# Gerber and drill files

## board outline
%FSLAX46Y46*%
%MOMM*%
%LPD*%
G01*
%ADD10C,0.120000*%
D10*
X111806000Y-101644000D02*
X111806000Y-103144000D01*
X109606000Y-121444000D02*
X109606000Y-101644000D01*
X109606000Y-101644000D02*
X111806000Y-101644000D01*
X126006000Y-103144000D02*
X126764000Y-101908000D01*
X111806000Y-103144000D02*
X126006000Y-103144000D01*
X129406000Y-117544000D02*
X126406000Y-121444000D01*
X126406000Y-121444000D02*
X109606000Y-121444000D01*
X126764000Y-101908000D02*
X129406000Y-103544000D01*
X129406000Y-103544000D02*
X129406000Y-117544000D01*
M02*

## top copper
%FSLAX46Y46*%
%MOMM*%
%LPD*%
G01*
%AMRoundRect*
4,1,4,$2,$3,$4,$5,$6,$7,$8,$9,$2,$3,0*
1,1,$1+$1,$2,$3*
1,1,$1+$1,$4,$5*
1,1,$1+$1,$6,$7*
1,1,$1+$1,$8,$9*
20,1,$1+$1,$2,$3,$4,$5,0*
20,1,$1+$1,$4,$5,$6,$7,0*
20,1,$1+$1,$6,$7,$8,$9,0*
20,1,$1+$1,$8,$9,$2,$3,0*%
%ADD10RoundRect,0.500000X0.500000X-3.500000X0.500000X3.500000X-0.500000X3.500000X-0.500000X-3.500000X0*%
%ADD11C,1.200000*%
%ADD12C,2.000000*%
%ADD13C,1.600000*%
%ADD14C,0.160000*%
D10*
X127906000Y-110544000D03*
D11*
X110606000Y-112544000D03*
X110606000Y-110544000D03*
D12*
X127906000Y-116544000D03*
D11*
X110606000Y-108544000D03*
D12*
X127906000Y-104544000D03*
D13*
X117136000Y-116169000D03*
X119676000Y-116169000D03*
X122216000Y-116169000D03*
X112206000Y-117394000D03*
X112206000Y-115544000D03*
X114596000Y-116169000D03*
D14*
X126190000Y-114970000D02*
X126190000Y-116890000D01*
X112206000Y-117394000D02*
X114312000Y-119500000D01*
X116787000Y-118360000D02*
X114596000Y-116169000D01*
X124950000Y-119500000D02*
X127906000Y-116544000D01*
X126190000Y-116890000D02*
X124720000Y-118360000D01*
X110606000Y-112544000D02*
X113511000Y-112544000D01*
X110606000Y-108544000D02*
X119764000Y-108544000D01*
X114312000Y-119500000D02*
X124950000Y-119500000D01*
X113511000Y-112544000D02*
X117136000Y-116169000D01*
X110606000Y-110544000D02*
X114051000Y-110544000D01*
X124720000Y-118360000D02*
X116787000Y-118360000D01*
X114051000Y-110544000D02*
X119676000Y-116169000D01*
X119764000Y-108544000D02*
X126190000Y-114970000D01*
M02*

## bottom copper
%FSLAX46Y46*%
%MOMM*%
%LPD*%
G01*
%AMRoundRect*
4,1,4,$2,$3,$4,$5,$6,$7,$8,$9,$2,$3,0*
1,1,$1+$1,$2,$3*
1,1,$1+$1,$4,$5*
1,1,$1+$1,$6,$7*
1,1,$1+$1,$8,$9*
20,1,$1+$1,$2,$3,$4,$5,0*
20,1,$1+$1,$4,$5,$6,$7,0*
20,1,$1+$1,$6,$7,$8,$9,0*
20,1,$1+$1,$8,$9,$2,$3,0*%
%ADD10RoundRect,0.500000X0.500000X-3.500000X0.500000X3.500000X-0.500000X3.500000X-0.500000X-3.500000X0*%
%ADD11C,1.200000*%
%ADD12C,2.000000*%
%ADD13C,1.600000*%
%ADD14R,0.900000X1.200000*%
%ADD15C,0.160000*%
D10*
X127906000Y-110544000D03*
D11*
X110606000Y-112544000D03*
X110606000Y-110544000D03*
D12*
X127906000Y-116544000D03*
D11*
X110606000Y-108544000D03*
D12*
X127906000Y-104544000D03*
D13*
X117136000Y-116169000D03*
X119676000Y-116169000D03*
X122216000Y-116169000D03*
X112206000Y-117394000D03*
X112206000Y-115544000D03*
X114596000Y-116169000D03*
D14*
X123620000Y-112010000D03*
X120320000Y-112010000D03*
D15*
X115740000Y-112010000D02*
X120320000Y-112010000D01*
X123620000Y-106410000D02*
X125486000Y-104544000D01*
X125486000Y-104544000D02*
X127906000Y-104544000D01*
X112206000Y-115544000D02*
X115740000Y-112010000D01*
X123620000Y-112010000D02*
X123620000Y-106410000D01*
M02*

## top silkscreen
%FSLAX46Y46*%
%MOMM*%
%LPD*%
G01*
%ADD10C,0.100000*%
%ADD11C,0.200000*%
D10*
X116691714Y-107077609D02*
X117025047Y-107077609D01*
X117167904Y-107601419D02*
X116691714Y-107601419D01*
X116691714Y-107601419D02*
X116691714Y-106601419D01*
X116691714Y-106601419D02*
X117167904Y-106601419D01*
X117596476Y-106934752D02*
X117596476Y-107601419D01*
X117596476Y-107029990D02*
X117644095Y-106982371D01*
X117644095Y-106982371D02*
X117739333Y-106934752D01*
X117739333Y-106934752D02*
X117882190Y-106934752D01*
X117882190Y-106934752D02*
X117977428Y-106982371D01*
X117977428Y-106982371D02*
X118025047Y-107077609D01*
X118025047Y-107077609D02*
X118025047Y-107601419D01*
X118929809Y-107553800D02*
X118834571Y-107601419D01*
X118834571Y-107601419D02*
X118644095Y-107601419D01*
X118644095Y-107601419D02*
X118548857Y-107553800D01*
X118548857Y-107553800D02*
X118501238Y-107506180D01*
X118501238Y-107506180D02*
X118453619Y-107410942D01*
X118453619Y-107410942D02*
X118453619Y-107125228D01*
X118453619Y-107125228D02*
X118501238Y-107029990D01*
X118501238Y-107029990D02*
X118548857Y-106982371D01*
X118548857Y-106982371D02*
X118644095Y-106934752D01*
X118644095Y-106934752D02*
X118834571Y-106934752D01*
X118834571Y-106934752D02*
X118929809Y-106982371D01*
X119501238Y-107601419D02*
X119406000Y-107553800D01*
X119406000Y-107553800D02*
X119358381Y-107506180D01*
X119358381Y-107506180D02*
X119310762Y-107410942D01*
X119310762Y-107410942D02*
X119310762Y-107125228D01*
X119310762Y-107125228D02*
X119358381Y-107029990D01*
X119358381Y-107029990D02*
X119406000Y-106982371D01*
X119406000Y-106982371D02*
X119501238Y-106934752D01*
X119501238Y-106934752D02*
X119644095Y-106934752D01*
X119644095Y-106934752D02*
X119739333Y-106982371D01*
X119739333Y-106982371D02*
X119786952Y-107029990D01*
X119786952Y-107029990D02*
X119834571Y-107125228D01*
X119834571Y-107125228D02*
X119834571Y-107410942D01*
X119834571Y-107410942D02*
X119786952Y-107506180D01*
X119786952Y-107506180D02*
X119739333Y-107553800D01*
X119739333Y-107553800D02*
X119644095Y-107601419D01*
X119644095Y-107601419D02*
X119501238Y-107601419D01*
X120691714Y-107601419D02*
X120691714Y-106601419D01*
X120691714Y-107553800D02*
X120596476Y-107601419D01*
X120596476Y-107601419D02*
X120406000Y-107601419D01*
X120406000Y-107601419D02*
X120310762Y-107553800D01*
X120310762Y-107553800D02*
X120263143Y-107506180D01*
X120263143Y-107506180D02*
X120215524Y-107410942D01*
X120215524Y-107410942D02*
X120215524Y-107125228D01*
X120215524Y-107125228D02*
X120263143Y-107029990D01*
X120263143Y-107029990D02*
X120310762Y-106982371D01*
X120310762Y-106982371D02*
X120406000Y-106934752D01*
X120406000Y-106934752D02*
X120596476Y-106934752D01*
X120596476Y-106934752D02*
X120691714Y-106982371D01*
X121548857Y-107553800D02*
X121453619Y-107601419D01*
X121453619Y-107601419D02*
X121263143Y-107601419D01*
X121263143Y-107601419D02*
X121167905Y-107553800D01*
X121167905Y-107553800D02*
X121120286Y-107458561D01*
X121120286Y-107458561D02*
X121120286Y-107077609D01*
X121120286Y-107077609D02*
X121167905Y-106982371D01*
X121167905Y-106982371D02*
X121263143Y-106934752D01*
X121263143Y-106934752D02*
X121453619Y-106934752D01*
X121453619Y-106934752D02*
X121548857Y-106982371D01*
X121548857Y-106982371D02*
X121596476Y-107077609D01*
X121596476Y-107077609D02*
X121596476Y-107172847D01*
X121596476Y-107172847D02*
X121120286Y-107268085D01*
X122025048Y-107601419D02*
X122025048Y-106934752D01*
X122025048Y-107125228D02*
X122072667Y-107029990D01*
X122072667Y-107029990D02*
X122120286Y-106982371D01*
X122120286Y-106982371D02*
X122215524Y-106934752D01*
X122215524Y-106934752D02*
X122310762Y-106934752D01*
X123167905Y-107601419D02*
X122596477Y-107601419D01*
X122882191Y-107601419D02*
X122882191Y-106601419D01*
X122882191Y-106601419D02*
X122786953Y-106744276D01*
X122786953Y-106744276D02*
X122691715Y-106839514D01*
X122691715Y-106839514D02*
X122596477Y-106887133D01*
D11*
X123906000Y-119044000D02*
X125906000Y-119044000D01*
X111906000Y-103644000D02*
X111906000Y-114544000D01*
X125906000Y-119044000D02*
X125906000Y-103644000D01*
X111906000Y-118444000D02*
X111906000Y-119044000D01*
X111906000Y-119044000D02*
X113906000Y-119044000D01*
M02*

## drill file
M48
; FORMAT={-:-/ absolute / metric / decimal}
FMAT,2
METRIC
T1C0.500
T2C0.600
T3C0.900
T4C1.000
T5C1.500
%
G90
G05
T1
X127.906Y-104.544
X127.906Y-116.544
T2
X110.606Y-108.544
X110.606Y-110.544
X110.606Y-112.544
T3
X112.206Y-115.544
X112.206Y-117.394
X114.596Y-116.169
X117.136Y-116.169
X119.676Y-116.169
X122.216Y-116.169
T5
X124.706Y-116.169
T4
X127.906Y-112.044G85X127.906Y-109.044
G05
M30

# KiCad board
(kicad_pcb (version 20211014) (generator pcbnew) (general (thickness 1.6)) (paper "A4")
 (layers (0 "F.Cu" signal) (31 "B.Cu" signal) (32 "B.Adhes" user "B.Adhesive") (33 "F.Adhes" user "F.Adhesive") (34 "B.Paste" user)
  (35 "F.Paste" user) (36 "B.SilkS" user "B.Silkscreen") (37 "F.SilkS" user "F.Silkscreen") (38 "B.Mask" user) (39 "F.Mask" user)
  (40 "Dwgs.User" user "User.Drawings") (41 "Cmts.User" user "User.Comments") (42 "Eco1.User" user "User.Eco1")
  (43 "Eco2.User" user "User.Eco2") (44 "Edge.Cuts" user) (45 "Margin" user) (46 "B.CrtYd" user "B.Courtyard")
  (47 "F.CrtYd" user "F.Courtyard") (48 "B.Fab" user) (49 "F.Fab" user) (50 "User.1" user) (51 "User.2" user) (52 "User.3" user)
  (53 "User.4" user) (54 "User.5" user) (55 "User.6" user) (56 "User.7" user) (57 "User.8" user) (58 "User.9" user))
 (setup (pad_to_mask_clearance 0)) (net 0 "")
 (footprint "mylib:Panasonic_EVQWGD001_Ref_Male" (layer "F.Cu") (at 119.906 110.544 90)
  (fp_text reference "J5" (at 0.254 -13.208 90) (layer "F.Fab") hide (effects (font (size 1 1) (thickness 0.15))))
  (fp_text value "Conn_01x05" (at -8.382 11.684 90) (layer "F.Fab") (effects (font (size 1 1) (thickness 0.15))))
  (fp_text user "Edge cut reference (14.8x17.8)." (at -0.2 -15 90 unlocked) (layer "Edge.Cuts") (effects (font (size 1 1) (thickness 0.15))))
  (fp_line (start 8.9 -8.1) (end 7.4 -8.1) (layer "Edge.Cuts") (width 0.12))
  (fp_line (start -10.9 -10.3) (end 8.9 -10.3) (layer "Edge.Cuts") (width 0.12))
  (fp_line (start 8.9 -10.3) (end 8.9 -8.1) (layer "Edge.Cuts") (width 0.12))
  (fp_line (start 7.4 6.1) (end 8.636 6.858) (layer "Edge.Cuts") (width 0.12))
  (fp_line (start 7.4 -8.1) (end 7.4 6.1) (layer "Edge.Cuts") (width 0.12))
  (fp_line (start -7 9.5) (end -10.9 6.5) (layer "Edge.Cuts") (width 0.12))
  (fp_line (start -10.9 6.5) (end -10.9 -10.3) (layer "Edge.Cuts") (width 0.12))
  (fp_line (start 8.636 6.858) (end 7 9.5) (layer "Edge.Cuts") (width 0.12))
  (fp_line (start 7 9.5) (end -7 9.5) (layer "Edge.Cuts") (width 0.12))
  (pad "" thru_hole roundrect (at 0 8 90) (size 8 2) (drill oval 4 1) (layers *.Cu *.Mask) (roundrect_rratio 0.25))
  (pad "a" thru_hole circle (at -2 -9.3 90) (size 1.2 1.2) (drill 0.6) (layers *.Cu *.Mask))
  (pad "b" thru_hole circle (at 0 -9.3 90) (size 1.2 1.2) (drill 0.6) (layers *.Cu *.Mask))
  (pad "col" thru_hole circle (at -6 8 90) (size 2 2) (drill 0.5) (layers *.Cu *.Mask))
  (pad "gnd" thru_hole circle (at 2 -9.3 90) (size 1.2 1.2) (drill 0.6) (layers *.Cu *.Mask))
  (pad "row" thru_hole circle (at 6 8 90) (size 2 2) (drill 0.5) (layers *.Cu *.Mask)))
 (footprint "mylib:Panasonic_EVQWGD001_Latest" (layer "F.Cu") (at 119.906 110.544 90)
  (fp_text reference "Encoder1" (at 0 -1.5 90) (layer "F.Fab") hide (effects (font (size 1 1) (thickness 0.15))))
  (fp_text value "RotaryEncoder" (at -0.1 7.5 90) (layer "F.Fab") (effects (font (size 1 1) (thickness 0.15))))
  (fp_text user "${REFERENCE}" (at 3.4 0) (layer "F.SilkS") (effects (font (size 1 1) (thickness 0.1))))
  (fp_line (start -8.5 4) (end -8.5 6) (layer "F.SilkS") (width 0.2))
  (fp_line (start 6.9 -8) (end -4 -8) (layer "F.SilkS") (width 0.2))
  (fp_line (start -8.5 6) (end 6.9 6) (layer "F.SilkS") (width 0.2))
  (fp_line (start -7.9 -8) (end -8.5 -8) (layer "F.SilkS") (width 0.2))
  (fp_line (start -8.5 -8) (end -8.5 -6) (layer "F.SilkS") (width 0.2))
  (pad "" np_thru_hole circle (at -5.625 4.8 90) (size 1.5 1.5) (drill 1.5) (layers *.Cu *.Mask))
  (pad "A" thru_hole circle (at -5.625 -2.77 90) (size 1.6 1.6) (drill 0.9) (layers *.Cu *.Mask))
  (pad "B" thru_hole circle (at -5.625 -0.23 90) (size 1.6 1.6) (drill 0.9) (layers *.Cu *.Mask))
  (pad "NC" thru_hole circle (at -5.625 2.31 90) (size 1.6 1.6) (drill 0.9) (layers *.Cu *.Mask))
  (pad "S1" thru_hole circle (at -6.85 -7.7 90) (size 1.6 1.6) (drill 0.9) (layers *.Cu *.Mask))
  (pad "S2" thru_hole circle (at -5 -7.7 90) (size 1.6 1.6) (drill 0.9) (layers *.Cu *.Mask))
  (pad "com" thru_hole circle (at -5.625 -5.31 90) (size 1.6 1.6) (drill 0.9) (layers *.Cu *.Mask)))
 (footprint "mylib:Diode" (layer "B.Cu") (at 121.97 112.01 180)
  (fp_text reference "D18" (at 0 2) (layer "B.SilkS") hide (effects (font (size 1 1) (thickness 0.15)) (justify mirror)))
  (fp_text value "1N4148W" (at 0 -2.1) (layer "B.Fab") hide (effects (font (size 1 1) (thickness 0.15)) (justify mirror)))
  (pad "1" smd rect (at -1.65 0 180) (size 0.9 1.2) (layers "B.Cu" "B.Paste" "B.Mask"))
  (pad "2" smd rect (at 1.65 0 180) (size 0.9 1.2) (layers "B.Cu" "B.Paste" "B.Mask")))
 (segment (start 126.19 114.97) (end 126.19 116.89) (width 0.16) (layer "F.Cu") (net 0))
 (segment (start 112.206 117.394) (end 114.312 119.5) (width 0.16) (layer "F.Cu") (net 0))
 (segment (start 116.787 118.36) (end 114.596 116.169) (width 0.16) (layer "F.Cu") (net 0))
 (segment (start 124.95 119.5) (end 127.906 116.544) (width 0.16) (layer "F.Cu") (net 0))
 (segment (start 126.19 116.89) (end 124.72 118.36) (width 0.16) (layer "F.Cu") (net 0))
 (segment (start 110.606 112.544) (end 113.511 112.544) (width 0.16) (layer "F.Cu") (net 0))
 (segment (start 110.606 108.544) (end 119.764 108.544) (width 0.16) (layer "F.Cu") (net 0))
 (segment (start 114.312 119.5) (end 124.95 119.5) (width 0.16) (layer "F.Cu") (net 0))
 (segment (start 113.511 112.544) (end 117.136 116.169) (width 0.16) (layer "F.Cu") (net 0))
 (segment (start 110.606 110.544) (end 114.051 110.544) (width 0.16) (layer "F.Cu") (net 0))
 (segment (start 124.72 118.36) (end 116.787 118.36) (width 0.16) (layer "F.Cu") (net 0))
 (segment (start 114.051 110.544) (end 119.676 116.169) (width 0.16) (layer "F.Cu") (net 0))
 (segment (start 119.764 108.544) (end 126.19 114.97) (width 0.16) (layer "F.Cu") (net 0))
 (segment (start 115.74 112.01) (end 120.32 112.01) (width 0.16) (layer "B.Cu") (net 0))
 (segment (start 123.62 106.41) (end 125.486 104.544) (width 0.16) (layer "B.Cu") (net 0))
 (segment (start 125.486 104.544) (end 127.906 104.544) (width 0.16) (layer "B.Cu") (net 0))
 (segment (start 112.206 115.544) (end 115.74 112.01) (width 0.16) (layer "B.Cu") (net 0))
 (segment (start 123.62 112.01) (end 123.62 106.41) (width 0.16) (layer "B.Cu") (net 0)))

